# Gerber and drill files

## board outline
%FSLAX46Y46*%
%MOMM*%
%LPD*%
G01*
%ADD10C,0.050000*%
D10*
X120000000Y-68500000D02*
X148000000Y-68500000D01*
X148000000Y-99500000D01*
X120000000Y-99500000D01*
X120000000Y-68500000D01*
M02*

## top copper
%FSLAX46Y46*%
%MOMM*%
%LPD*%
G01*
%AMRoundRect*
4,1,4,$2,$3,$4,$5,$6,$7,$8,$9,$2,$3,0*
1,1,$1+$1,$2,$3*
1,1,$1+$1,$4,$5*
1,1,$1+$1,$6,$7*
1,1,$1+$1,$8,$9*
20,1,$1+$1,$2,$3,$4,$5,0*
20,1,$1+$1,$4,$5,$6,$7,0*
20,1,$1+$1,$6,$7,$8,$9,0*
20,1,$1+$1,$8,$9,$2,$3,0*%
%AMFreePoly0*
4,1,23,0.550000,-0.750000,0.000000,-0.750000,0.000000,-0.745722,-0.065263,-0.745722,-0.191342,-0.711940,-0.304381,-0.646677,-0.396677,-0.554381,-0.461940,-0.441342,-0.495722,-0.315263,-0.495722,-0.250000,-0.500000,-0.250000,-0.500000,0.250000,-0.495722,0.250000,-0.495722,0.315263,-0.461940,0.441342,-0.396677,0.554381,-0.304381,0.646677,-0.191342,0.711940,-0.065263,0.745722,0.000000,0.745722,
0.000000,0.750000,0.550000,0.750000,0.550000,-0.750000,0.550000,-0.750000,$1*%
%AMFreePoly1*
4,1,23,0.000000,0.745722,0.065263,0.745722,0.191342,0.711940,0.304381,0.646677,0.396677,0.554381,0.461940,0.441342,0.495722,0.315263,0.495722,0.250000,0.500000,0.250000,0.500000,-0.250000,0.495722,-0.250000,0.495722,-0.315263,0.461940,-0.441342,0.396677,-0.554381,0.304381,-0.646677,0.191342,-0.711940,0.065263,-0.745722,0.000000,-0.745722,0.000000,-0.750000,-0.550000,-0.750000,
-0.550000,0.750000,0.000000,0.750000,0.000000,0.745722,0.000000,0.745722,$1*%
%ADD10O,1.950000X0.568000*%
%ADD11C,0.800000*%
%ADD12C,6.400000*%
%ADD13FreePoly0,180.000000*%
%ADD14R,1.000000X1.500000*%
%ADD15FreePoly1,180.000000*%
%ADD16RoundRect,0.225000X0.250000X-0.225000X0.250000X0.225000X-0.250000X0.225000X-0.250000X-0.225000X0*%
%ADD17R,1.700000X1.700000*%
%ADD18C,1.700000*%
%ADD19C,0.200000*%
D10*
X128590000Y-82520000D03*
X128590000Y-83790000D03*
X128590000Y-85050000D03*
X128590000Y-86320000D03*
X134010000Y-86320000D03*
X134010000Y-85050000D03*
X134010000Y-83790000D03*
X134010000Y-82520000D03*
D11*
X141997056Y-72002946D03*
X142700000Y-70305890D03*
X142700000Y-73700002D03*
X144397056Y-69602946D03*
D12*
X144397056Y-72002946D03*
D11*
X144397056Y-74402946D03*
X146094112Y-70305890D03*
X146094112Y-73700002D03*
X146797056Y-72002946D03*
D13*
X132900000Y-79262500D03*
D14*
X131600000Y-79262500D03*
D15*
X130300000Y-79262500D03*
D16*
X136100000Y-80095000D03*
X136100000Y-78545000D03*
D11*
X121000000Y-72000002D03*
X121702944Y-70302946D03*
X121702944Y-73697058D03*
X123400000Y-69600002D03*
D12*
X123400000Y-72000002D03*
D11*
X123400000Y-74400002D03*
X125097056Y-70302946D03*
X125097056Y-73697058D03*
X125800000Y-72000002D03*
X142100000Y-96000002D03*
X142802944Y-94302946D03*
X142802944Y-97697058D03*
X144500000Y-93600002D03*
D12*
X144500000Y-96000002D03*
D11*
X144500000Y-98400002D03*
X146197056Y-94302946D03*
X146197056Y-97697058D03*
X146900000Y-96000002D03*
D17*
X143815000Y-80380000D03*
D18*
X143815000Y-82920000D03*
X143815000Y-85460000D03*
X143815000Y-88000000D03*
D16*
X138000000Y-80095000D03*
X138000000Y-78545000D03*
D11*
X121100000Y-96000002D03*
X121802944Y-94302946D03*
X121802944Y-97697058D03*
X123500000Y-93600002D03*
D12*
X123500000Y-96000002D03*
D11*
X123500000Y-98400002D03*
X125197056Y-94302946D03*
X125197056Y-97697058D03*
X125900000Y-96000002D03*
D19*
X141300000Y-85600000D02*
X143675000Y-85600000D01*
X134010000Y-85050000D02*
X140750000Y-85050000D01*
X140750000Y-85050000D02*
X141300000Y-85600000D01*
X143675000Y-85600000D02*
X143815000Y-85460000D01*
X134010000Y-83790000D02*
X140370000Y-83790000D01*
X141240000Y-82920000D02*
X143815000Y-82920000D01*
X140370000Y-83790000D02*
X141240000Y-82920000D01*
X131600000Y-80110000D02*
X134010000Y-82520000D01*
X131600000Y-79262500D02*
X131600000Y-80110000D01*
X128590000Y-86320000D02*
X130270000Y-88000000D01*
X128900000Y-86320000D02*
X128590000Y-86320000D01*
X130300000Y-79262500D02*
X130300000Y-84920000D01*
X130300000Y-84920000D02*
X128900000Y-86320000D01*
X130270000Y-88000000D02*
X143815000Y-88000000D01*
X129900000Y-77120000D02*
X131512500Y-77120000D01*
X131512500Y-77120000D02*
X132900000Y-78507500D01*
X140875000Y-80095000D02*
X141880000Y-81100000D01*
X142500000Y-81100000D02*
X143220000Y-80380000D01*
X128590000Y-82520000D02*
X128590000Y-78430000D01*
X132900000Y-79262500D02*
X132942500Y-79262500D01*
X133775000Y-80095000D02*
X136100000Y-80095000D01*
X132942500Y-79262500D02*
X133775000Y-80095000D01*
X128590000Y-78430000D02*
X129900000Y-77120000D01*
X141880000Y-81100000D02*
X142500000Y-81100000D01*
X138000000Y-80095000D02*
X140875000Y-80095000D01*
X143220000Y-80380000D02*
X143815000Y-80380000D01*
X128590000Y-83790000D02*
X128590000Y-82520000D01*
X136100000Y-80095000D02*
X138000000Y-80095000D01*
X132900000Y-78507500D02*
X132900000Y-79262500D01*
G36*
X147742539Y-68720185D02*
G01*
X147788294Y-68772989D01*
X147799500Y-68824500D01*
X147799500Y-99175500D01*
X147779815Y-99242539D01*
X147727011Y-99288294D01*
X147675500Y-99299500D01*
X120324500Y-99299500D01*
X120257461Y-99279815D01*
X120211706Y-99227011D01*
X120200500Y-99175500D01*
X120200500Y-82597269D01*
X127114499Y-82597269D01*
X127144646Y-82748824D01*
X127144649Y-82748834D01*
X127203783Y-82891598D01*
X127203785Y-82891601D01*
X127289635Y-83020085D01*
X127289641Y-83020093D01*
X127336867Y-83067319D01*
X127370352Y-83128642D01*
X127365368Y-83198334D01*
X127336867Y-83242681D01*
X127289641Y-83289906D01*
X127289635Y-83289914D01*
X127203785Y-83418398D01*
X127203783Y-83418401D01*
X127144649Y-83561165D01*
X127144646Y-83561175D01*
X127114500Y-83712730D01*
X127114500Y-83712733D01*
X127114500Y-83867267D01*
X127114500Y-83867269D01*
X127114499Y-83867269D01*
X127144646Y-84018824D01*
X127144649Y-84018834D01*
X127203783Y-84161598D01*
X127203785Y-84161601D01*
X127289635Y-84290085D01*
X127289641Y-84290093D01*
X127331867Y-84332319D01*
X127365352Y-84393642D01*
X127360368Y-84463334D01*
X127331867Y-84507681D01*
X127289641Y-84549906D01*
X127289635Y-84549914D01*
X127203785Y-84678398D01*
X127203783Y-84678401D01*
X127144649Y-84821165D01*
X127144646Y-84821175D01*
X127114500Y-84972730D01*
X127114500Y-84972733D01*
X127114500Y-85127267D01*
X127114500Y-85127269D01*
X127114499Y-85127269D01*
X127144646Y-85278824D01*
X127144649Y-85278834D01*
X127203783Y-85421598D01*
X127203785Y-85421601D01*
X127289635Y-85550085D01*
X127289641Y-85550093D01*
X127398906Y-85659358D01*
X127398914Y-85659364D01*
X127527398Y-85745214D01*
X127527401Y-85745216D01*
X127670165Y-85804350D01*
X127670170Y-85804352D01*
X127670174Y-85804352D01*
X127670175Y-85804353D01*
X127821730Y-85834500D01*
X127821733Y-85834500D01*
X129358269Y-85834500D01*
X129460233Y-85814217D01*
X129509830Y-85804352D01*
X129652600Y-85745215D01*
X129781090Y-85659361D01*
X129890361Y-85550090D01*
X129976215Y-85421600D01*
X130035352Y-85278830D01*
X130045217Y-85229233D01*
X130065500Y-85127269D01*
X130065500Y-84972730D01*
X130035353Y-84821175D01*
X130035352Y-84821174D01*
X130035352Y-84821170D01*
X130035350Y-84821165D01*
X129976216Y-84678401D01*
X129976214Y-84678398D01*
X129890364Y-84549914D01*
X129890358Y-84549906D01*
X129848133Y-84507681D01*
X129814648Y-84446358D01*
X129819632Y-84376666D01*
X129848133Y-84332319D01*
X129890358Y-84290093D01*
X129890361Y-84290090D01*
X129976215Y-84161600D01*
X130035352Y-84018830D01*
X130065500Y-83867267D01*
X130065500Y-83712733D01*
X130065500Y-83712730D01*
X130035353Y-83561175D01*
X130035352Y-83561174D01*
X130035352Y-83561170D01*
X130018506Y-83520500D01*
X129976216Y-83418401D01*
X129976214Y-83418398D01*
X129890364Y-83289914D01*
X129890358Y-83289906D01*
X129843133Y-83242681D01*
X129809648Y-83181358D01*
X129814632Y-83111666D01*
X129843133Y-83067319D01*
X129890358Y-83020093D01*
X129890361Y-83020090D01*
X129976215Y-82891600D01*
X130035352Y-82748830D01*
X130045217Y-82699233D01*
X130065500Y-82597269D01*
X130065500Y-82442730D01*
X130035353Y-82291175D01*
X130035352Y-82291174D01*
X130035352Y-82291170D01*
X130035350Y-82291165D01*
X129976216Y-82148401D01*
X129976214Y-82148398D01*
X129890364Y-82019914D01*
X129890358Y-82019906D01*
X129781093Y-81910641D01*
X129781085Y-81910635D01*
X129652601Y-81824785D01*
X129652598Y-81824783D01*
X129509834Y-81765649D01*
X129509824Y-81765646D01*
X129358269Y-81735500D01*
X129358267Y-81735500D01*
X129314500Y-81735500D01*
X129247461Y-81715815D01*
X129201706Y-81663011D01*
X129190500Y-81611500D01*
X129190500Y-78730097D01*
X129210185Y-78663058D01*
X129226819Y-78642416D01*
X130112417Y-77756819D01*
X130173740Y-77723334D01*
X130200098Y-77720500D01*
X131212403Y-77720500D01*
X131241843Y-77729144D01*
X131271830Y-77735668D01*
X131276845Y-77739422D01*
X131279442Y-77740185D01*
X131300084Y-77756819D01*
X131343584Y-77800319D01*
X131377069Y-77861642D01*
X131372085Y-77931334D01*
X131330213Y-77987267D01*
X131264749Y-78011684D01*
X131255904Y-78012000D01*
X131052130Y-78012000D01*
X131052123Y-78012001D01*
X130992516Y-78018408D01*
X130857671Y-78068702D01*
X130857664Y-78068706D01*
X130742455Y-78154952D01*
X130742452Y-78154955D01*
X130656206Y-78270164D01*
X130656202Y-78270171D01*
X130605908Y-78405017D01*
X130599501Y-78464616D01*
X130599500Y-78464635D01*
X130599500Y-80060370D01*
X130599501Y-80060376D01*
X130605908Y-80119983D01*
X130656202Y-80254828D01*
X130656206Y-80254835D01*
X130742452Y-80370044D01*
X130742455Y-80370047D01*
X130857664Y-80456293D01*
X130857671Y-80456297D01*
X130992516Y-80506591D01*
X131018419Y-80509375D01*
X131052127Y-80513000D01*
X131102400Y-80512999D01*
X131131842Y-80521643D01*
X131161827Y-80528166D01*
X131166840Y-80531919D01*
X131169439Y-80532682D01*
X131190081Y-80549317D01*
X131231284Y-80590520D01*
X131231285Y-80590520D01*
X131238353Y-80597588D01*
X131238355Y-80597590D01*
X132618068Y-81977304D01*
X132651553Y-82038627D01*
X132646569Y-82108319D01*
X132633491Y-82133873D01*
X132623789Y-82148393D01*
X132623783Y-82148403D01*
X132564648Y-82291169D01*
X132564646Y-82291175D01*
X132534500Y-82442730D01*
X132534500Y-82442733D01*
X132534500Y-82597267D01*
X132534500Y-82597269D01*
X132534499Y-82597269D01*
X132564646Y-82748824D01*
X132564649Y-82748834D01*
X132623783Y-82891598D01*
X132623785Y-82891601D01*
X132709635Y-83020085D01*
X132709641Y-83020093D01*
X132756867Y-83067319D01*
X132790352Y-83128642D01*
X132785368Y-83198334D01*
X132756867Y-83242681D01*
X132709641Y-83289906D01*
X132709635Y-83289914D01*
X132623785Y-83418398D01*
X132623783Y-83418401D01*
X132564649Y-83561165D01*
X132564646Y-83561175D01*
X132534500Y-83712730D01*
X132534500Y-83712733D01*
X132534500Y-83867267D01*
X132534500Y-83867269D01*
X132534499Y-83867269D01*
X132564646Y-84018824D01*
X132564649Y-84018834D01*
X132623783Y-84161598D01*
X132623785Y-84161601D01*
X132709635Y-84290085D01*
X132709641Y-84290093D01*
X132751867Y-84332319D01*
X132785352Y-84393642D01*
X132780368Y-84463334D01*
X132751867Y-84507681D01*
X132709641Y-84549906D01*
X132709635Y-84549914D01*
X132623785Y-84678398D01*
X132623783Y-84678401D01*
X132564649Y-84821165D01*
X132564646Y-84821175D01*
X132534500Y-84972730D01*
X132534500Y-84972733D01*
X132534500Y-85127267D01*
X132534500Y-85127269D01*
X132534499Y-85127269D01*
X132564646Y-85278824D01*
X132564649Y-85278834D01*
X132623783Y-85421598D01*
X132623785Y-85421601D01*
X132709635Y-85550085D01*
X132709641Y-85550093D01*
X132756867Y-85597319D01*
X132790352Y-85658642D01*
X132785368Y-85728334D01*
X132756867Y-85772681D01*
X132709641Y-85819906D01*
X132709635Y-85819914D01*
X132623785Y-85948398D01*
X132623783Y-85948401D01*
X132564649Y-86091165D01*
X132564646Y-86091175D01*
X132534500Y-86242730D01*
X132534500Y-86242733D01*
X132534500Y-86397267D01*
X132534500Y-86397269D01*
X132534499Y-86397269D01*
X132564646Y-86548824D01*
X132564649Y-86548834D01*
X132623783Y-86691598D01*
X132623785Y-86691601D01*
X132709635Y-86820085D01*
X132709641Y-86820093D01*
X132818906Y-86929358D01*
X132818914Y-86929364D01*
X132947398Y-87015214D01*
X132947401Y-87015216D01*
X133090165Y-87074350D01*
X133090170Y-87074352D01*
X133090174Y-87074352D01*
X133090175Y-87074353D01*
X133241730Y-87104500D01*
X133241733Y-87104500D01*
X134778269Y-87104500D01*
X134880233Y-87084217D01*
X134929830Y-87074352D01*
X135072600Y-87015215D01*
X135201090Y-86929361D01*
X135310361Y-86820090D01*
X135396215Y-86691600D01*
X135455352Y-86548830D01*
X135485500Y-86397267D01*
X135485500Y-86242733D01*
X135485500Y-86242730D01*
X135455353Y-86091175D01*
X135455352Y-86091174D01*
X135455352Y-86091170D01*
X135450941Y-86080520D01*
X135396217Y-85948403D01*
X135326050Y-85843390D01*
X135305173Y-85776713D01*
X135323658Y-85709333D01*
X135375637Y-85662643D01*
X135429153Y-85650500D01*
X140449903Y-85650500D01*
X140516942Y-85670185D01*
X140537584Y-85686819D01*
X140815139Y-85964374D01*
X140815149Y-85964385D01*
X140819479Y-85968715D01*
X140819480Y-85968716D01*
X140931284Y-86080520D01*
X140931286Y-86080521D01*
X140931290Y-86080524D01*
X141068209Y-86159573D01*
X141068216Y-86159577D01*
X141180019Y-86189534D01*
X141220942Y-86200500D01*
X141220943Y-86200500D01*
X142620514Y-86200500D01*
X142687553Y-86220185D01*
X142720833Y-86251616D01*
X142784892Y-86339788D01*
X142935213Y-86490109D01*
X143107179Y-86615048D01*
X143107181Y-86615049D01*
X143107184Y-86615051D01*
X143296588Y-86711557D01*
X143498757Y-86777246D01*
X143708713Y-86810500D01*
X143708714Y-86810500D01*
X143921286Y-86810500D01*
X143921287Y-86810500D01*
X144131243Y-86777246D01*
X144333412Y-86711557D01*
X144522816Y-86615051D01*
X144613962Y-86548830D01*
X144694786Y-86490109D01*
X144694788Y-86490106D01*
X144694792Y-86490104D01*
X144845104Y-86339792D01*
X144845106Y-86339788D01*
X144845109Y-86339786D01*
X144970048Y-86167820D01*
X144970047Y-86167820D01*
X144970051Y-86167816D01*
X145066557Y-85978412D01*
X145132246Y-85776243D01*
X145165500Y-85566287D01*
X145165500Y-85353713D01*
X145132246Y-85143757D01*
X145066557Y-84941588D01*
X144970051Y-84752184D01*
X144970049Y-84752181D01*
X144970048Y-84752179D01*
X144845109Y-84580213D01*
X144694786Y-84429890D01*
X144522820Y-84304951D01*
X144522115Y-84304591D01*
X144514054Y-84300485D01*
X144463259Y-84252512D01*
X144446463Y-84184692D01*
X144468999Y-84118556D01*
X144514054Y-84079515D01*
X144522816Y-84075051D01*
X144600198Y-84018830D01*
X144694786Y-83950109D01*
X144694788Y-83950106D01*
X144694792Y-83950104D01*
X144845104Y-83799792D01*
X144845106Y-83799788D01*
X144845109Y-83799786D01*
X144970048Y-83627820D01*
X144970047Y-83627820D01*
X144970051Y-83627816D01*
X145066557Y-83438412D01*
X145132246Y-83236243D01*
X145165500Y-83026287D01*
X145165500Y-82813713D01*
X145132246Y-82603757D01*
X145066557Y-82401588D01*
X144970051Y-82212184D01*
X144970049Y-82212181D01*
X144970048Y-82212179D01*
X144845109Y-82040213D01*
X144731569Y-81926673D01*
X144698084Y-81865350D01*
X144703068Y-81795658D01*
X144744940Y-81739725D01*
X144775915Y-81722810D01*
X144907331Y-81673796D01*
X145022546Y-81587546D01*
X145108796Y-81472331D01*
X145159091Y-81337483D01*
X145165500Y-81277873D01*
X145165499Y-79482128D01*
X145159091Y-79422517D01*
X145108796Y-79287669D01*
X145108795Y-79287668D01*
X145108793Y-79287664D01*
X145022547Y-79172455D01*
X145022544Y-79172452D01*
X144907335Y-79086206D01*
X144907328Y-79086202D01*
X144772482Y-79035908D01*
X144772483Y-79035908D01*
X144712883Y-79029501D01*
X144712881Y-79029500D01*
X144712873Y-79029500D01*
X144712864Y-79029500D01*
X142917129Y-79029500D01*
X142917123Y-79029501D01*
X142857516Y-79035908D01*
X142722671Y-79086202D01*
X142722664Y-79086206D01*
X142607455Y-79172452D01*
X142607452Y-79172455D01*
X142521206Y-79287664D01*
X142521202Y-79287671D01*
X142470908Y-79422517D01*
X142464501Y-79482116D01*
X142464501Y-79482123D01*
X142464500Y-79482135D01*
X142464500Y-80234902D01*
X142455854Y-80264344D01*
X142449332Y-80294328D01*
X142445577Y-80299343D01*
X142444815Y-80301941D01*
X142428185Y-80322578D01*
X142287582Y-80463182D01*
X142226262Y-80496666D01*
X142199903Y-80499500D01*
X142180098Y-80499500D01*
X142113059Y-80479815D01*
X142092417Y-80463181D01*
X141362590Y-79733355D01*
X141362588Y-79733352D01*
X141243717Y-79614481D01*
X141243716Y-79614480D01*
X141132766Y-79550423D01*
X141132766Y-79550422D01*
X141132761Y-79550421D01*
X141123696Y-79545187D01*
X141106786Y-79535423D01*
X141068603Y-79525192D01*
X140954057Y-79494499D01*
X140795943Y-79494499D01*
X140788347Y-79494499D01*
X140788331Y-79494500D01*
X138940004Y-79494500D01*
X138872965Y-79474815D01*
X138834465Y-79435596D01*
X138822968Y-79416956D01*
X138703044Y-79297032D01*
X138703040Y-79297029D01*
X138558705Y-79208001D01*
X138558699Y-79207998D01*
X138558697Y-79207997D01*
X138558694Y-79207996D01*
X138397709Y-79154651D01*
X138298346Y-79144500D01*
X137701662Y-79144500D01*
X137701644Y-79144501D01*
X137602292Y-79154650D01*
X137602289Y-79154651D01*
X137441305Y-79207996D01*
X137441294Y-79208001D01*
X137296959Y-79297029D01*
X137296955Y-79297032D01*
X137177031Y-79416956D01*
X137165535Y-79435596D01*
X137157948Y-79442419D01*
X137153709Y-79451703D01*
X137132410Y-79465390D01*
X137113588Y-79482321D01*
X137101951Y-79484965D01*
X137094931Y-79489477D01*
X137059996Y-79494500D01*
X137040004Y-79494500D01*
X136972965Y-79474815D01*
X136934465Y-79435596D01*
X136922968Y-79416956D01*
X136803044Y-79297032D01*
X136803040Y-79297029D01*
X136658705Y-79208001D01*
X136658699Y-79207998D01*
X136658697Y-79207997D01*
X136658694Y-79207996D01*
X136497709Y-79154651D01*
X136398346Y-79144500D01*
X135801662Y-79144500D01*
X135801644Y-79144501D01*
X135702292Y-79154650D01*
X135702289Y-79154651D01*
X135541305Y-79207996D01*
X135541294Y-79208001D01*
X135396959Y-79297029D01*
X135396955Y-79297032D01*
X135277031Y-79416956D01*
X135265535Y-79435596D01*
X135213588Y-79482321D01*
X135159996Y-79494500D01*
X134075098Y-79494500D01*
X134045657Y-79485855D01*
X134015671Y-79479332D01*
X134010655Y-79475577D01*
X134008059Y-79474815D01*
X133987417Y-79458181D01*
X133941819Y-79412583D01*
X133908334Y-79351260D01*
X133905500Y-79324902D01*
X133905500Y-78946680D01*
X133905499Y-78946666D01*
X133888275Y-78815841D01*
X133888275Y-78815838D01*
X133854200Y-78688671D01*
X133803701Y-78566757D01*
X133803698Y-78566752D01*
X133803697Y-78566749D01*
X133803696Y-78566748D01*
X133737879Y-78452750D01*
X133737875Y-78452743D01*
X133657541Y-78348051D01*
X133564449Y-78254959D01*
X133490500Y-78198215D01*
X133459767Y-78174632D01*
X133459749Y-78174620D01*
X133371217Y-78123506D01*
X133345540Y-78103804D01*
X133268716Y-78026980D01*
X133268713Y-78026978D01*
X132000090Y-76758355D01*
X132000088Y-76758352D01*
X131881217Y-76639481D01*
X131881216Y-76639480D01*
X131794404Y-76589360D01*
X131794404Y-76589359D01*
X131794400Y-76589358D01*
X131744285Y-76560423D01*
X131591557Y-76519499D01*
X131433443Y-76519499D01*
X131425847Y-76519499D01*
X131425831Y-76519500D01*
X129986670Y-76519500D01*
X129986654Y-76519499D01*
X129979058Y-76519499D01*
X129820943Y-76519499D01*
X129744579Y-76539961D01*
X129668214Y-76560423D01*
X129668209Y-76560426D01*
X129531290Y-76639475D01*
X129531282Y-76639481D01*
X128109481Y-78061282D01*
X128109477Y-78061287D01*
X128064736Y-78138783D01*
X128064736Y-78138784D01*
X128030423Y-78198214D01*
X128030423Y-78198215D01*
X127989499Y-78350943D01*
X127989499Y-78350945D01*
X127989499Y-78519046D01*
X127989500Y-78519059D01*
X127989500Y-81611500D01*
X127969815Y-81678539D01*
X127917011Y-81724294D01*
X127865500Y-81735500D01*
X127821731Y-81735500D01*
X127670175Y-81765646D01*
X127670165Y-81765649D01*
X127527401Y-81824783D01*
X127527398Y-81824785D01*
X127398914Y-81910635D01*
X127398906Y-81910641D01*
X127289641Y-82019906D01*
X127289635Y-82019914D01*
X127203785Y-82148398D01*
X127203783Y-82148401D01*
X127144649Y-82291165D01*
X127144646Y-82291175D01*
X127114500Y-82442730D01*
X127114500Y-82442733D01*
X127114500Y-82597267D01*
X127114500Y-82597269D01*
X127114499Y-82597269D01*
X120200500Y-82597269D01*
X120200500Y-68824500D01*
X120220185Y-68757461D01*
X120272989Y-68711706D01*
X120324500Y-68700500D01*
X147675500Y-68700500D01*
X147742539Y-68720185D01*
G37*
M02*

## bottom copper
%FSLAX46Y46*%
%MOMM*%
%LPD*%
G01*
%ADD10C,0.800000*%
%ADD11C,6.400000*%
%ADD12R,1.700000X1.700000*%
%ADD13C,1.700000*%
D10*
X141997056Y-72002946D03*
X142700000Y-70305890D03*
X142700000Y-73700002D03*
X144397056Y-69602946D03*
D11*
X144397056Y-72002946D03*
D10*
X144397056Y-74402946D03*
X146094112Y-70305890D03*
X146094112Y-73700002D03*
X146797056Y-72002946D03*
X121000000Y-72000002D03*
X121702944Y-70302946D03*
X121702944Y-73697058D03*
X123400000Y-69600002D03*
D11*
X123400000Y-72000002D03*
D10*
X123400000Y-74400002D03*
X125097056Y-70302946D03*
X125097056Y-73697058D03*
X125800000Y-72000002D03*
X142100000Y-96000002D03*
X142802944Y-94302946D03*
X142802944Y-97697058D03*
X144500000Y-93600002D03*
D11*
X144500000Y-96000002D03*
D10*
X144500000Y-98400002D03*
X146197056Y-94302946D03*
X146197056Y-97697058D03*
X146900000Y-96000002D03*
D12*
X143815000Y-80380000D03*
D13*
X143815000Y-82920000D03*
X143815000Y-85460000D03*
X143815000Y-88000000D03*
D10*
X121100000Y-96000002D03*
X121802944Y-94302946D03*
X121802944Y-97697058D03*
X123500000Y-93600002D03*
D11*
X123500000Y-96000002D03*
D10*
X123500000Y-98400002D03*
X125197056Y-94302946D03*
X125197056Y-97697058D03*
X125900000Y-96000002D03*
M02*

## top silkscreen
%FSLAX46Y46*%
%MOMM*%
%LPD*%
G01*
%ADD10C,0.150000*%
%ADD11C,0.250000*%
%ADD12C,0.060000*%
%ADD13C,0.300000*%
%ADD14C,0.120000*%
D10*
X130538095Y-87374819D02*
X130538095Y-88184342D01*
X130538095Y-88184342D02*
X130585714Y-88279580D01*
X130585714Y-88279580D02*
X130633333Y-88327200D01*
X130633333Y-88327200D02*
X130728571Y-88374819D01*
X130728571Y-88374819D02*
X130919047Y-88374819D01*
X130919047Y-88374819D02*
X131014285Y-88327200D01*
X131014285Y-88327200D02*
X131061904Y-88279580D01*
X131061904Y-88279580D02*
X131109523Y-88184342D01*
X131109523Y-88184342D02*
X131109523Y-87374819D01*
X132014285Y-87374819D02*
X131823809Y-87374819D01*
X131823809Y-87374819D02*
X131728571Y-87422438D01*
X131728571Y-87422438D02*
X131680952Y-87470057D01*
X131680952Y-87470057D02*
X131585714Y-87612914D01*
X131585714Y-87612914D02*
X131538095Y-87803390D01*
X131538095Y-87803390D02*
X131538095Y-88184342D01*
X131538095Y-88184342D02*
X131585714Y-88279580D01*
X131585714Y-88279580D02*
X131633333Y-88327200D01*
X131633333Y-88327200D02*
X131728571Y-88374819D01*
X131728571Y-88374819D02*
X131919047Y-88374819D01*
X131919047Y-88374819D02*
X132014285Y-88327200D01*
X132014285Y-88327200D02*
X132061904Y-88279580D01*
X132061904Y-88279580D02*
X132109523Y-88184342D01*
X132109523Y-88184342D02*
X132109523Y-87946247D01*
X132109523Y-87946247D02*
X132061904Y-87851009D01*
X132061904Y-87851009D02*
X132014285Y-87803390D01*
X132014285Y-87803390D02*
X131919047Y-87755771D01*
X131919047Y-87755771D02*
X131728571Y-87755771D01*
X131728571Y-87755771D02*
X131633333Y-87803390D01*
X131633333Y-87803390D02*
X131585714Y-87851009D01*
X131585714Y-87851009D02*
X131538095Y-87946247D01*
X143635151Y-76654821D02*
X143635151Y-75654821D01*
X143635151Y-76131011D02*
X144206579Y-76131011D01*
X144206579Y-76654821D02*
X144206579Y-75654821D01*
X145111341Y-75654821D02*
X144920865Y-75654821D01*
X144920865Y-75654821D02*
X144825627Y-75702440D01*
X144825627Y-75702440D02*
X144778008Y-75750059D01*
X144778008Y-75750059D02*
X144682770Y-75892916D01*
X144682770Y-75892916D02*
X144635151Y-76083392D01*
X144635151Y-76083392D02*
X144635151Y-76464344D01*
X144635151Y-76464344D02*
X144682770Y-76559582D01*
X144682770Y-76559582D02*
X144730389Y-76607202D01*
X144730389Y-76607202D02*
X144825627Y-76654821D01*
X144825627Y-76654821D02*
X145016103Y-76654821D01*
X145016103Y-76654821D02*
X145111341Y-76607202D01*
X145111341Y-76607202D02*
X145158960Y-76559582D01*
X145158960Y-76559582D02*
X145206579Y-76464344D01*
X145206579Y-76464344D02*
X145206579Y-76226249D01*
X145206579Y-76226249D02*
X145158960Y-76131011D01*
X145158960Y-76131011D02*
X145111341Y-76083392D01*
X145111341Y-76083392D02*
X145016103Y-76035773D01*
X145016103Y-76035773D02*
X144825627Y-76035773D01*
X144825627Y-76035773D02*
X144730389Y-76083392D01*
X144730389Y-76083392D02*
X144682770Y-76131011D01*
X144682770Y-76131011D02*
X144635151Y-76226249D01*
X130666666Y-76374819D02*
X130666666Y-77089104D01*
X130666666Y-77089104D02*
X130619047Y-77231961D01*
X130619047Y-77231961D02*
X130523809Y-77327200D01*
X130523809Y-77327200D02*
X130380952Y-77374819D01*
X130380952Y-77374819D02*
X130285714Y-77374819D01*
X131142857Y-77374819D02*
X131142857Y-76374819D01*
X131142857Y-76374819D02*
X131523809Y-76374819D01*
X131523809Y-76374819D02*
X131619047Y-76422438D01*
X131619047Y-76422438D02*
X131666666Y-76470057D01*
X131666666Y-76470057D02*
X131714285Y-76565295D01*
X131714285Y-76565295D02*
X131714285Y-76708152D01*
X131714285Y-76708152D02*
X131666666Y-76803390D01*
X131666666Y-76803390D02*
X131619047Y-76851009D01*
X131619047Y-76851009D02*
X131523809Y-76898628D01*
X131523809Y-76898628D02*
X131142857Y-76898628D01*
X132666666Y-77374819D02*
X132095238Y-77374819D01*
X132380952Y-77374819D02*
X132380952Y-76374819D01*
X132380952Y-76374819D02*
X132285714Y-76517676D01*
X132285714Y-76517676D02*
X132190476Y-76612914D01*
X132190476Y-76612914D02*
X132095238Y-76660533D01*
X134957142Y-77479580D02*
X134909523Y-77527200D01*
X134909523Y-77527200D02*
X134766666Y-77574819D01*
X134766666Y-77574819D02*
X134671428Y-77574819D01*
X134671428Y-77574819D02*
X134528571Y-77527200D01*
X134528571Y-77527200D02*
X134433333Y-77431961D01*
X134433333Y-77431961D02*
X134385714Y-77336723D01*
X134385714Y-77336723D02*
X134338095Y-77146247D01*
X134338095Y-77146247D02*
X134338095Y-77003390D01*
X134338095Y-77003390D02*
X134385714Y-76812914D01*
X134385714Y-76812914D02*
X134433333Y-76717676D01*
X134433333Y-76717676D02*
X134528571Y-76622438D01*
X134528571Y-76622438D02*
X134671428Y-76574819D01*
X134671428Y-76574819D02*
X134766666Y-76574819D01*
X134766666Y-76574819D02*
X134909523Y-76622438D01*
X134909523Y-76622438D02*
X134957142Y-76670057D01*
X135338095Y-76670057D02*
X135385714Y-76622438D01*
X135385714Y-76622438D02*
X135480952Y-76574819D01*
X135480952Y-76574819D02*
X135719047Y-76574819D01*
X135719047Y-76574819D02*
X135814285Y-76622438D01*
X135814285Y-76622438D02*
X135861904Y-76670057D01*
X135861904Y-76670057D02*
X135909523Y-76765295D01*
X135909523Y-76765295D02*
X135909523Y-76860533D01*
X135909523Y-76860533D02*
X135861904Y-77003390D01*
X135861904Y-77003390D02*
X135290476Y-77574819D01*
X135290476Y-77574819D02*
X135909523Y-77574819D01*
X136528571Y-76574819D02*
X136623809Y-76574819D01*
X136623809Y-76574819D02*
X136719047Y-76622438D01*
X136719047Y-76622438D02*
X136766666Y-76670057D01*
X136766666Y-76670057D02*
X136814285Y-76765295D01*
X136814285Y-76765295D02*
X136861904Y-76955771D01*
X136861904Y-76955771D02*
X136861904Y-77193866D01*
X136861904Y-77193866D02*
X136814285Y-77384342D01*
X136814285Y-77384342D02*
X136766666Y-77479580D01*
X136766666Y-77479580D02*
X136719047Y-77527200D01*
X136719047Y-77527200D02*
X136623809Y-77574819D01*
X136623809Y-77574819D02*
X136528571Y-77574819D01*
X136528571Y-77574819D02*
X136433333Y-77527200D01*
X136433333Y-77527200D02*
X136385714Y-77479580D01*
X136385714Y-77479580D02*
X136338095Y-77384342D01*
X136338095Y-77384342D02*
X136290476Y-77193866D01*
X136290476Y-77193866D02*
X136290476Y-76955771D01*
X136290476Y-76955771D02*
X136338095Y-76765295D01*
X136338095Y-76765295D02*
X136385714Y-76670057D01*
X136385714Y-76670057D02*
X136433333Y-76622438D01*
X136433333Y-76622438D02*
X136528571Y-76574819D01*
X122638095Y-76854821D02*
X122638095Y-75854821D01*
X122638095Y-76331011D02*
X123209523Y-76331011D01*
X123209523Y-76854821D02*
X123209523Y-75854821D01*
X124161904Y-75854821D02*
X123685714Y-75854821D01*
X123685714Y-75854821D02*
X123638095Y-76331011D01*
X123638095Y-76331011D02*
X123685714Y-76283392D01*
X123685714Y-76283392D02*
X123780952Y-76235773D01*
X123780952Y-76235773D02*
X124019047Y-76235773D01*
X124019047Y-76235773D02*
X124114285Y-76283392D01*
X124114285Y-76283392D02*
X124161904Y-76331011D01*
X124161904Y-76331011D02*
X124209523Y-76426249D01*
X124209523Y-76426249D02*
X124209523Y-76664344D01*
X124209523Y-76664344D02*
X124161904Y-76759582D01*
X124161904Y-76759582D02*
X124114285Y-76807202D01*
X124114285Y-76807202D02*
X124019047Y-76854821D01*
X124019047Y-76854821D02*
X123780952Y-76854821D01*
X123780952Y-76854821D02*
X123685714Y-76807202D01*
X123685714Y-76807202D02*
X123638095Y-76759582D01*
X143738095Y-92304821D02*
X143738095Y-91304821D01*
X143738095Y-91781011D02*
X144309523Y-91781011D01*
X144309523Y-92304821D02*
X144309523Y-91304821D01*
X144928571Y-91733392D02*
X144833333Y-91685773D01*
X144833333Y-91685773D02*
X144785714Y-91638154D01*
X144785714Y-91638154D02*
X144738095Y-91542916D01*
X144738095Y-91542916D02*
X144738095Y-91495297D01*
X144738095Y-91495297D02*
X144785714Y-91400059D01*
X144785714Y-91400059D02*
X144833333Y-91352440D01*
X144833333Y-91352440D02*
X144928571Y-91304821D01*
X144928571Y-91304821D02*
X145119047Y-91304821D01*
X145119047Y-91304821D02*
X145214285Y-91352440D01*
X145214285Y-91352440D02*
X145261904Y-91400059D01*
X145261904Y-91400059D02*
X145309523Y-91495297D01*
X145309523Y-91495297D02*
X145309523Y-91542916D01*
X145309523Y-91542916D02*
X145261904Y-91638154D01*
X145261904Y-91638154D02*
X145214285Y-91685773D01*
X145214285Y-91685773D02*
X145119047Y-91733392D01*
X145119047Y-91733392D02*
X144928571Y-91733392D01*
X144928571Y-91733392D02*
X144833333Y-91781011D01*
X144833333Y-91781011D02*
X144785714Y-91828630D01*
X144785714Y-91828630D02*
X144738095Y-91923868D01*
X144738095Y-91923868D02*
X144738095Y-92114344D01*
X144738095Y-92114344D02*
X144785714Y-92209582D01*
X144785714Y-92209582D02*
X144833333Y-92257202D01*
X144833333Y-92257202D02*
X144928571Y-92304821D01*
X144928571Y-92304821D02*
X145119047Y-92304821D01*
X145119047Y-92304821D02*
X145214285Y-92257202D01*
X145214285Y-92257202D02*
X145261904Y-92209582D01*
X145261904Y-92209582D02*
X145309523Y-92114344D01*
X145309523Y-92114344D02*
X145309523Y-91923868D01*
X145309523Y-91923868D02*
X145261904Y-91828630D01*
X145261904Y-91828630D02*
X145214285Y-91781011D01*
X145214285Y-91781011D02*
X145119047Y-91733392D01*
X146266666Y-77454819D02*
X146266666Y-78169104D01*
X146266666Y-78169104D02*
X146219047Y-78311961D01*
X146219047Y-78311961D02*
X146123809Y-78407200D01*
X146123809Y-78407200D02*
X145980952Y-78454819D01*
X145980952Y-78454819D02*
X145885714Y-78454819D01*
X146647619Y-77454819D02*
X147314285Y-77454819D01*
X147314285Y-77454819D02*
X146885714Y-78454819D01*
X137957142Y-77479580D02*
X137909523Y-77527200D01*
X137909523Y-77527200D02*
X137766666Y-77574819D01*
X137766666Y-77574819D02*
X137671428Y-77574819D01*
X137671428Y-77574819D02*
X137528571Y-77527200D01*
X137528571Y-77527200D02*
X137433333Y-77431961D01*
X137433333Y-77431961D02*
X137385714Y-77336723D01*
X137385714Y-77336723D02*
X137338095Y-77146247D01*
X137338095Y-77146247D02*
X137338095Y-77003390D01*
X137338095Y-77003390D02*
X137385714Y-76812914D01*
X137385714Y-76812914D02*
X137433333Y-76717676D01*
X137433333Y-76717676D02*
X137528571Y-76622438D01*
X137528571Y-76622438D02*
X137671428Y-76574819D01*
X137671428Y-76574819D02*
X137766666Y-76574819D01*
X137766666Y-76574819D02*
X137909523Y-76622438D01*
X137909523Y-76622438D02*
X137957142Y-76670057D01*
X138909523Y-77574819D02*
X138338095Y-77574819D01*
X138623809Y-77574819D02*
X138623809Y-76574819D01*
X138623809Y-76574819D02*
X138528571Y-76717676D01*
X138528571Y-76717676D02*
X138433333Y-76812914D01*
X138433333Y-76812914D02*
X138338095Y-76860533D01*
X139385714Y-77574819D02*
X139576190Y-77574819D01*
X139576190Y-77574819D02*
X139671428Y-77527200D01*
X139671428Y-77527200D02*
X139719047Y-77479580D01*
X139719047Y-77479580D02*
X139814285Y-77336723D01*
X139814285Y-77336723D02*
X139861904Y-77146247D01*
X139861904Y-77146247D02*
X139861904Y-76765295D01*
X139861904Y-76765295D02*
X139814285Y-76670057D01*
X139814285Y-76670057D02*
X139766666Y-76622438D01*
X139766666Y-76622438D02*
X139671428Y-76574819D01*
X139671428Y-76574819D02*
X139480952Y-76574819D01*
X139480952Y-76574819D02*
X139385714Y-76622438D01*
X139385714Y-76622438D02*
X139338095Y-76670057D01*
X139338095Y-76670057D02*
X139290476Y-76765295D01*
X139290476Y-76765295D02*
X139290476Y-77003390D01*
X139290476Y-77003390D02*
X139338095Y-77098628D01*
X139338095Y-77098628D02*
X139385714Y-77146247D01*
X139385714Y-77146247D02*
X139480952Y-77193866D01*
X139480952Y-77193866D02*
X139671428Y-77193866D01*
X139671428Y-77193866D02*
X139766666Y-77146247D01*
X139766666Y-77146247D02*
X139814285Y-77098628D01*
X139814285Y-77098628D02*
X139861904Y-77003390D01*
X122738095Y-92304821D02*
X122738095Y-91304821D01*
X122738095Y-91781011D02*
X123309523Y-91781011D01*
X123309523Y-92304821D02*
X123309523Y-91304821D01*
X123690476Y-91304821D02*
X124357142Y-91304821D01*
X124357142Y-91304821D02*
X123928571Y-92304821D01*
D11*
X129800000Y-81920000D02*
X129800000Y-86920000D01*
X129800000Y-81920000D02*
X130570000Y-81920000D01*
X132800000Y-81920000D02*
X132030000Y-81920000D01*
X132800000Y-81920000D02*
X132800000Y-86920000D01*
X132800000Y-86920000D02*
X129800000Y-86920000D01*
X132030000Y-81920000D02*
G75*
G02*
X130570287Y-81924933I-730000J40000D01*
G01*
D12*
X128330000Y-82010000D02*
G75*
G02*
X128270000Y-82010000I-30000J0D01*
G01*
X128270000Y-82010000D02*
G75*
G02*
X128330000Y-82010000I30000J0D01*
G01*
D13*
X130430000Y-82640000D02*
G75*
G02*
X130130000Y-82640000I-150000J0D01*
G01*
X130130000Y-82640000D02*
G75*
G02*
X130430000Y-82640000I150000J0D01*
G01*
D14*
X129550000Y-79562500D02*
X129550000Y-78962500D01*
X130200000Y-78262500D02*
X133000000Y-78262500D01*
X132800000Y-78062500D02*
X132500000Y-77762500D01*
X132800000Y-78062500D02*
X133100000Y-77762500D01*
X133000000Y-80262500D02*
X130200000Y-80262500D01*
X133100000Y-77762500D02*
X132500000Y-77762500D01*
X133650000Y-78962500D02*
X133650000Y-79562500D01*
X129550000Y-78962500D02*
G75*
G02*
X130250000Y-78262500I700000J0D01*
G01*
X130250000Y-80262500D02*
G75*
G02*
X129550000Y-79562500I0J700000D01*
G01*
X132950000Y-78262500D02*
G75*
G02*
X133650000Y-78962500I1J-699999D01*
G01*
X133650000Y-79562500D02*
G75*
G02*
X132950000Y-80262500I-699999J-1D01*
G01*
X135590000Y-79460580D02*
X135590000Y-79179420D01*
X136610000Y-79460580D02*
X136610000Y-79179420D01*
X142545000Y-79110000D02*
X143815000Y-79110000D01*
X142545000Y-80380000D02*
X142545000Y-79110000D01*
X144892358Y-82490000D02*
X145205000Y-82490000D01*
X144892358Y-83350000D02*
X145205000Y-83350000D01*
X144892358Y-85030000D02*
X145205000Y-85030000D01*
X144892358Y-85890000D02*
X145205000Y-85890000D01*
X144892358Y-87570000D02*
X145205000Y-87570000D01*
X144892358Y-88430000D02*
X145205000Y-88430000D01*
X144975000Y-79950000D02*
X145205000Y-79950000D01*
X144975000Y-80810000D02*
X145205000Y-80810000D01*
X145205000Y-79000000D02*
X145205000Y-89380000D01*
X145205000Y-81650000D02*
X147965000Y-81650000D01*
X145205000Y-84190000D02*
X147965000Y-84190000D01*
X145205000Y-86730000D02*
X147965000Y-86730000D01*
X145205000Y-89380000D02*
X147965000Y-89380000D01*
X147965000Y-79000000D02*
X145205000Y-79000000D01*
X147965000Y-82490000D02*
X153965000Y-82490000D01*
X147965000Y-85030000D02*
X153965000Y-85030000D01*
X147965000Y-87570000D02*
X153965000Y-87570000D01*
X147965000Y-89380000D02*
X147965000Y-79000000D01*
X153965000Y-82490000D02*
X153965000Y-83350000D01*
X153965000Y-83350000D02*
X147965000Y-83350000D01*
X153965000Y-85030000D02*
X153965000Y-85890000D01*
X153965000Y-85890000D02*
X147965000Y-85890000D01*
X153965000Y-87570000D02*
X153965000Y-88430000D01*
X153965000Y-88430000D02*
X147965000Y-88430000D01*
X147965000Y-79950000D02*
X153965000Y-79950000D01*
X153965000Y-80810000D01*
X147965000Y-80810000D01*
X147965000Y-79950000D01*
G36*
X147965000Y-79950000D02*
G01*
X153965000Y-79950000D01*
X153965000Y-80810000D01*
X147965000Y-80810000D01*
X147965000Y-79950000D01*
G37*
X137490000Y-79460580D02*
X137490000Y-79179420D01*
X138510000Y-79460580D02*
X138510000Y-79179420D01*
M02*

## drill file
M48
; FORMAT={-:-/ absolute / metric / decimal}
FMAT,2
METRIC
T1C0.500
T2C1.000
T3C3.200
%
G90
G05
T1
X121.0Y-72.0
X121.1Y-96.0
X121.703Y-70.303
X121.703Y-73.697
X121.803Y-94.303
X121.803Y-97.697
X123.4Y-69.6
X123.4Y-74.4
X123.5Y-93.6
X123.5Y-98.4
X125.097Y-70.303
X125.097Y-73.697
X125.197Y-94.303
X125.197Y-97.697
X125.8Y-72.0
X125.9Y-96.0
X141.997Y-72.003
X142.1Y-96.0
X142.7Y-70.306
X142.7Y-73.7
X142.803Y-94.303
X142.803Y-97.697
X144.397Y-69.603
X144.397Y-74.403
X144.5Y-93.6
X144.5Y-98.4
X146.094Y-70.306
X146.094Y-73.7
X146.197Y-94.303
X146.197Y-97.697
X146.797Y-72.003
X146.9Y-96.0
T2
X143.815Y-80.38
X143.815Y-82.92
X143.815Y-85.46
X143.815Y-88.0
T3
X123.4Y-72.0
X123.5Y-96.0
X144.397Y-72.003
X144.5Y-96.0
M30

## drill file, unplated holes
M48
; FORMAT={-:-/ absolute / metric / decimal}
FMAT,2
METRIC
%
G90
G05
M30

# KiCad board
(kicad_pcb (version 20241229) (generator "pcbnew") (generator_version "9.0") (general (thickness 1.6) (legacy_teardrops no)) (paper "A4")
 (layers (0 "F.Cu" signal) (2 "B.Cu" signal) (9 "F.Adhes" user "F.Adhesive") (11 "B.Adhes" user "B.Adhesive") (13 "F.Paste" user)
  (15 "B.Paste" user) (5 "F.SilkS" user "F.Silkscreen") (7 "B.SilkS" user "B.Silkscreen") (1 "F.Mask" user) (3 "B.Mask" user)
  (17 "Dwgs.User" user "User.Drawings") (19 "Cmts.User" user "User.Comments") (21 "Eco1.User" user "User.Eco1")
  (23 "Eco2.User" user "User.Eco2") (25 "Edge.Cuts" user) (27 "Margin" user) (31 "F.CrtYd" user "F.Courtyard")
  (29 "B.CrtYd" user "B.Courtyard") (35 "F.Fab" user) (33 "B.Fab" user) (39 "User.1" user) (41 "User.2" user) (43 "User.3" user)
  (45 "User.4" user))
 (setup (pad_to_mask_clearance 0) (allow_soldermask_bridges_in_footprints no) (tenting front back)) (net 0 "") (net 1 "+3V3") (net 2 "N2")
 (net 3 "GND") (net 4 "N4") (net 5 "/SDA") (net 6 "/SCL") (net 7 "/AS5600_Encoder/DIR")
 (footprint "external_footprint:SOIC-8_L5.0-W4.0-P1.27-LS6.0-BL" (layer "F.Cu") (at 131.3 84.42 -90)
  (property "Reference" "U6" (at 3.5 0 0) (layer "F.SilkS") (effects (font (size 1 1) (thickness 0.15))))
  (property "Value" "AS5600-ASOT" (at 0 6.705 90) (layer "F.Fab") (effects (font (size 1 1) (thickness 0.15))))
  (fp_line (start -2.5 1.5) (end 2.5 1.5) (stroke (width 0.25) (type solid)) (layer "F.SilkS"))
  (fp_line (start -2.5 1.5) (end -2.5 0.73) (stroke (width 0.25) (type solid)) (layer "F.SilkS"))
  (fp_line (start -2.5 -1.5) (end -2.5 -0.73) (stroke (width 0.25) (type solid)) (layer "F.SilkS"))
  (fp_line (start -2.5 -1.5) (end 2.5 -1.5) (stroke (width 0.25) (type solid)) (layer "F.SilkS"))
  (fp_line (start 2.5 -1.5) (end 2.5 1.5) (stroke (width 0.25) (type solid)) (layer "F.SilkS"))
  (fp_arc (start -2.5 -0.73) (mid -1.808909 -0.002471) (end -2.495067 0.729713) (stroke (width 0.25) (type solid)) (layer "F.SilkS"))
  (fp_circle (center -2.41 3) (end -2.38 3) (stroke (width 0.06) (type solid)) (fill no) (layer "F.SilkS"))
  (fp_circle (center -1.78 1.02) (end -1.63 1.02) (stroke (width 0.3) (type solid)) (fill no) (layer "F.SilkS"))
  (pad "1" smd oval (at -1.9 2.71 270) (size 0.568 1.95) (layers "F.Cu" "F.Mask" "F.Paste") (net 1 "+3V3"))
  (pad "2" smd oval (at -0.63 2.71 270) (size 0.568 1.95) (layers "F.Cu" "F.Mask" "F.Paste") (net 1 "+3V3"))
  (pad "3" smd oval (at 0.63 2.71 270) (size 0.568 1.95) (layers "F.Cu" "F.Mask" "F.Paste") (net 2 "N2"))
  (pad "4" smd oval (at 1.9 2.71 270) (size 0.568 1.95) (layers "F.Cu" "F.Mask" "F.Paste") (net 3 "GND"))
  (pad "5" smd oval (at 1.9 -2.71 270) (size 0.568 1.95) (layers "F.Cu" "F.Mask" "F.Paste") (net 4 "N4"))
  (pad "6" smd oval (at 0.63 -2.71 270) (size 0.568 1.95) (layers "F.Cu" "F.Mask" "F.Paste") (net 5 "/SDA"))
  (pad "7" smd oval (at -0.63 -2.71 270) (size 0.568 1.95) (layers "F.Cu" "F.Mask" "F.Paste") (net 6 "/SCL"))
  (pad "8" smd oval (at -1.9 -2.71 270) (size 0.568 1.95) (layers "F.Cu" "F.Mask" "F.Paste") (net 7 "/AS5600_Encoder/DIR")))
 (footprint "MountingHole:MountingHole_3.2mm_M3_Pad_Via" (layer "F.Cu") (at 144.397056 72.002946)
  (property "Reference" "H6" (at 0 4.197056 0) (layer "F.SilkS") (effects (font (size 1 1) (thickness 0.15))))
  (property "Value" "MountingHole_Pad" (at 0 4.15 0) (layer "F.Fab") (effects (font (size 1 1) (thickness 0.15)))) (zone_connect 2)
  (pad "1" thru_hole circle (at -2.4 0) (size 0.8 0.8) (drill 0.5) (layers "*.Cu" "*.Mask") (remove_unused_layers no) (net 3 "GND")
   (zone_connect 2))
  (pad "1" thru_hole circle (at -1.697056 -1.697056) (size 0.8 0.8) (drill 0.5) (layers "*.Cu" "*.Mask") (remove_unused_layers no)
   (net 3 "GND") (zone_connect 2))
  (pad "1" thru_hole circle (at -1.697056 1.697056) (size 0.8 0.8) (drill 0.5) (layers "*.Cu" "*.Mask") (remove_unused_layers no)
   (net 3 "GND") (zone_connect 2))
  (pad "1" thru_hole circle (at 0 -2.4) (size 0.8 0.8) (drill 0.5) (layers "*.Cu" "*.Mask") (remove_unused_layers no) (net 3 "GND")
   (zone_connect 2))
  (pad "1" thru_hole circle (at 0 0) (size 6.4 6.4) (drill 3.2) (layers "*.Cu" "*.Mask") (remove_unused_layers no) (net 3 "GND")
   (zone_connect 2))
  (pad "1" thru_hole circle (at 0 2.4) (size 0.8 0.8) (drill 0.5) (layers "*.Cu" "*.Mask") (remove_unused_layers no) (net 3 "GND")
   (zone_connect 2))
  (pad "1" thru_hole circle (at 1.697056 -1.697056) (size 0.8 0.8) (drill 0.5) (layers "*.Cu" "*.Mask") (remove_unused_layers no)
   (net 3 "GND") (zone_connect 2))
  (pad "1" thru_hole circle (at 1.697056 1.697056) (size 0.8 0.8) (drill 0.5) (layers "*.Cu" "*.Mask") (remove_unused_layers no)
   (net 3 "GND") (zone_connect 2))
  (pad "1" thru_hole circle (at 2.4 0) (size 0.8 0.8) (drill 0.5) (layers "*.Cu" "*.Mask") (remove_unused_layers no) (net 3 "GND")
   (zone_connect 2)))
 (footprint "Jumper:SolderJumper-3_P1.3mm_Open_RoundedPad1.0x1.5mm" (layer "F.Cu") (at 131.6 79.2625 180)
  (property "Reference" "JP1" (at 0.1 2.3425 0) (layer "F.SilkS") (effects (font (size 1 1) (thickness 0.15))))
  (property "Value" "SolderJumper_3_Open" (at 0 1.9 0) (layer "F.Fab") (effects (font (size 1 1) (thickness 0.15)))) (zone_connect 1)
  (fp_line (start 2.05 -0.3) (end 2.05 0.3) (stroke (width 0.12) (type solid)) (layer "F.SilkS"))
  (fp_line (start 1.4 1) (end -1.4 1) (stroke (width 0.12) (type solid)) (layer "F.SilkS"))
  (fp_line (start -1.2 1.2) (end -0.9 1.5) (stroke (width 0.12) (type solid)) (layer "F.SilkS"))
  (fp_line (start -1.2 1.2) (end -1.5 1.5) (stroke (width 0.12) (type solid)) (layer "F.SilkS"))
  (fp_line (start -1.4 -1) (end 1.4 -1) (stroke (width 0.12) (type solid)) (layer "F.SilkS"))
  (fp_line (start -1.5 1.5) (end -0.9 1.5) (stroke (width 0.12) (type solid)) (layer "F.SilkS"))
  (fp_line (start -2.05 0.3) (end -2.05 -0.3) (stroke (width 0.12) (type solid)) (layer "F.SilkS"))
  (fp_arc (start 2.05 0.3) (mid 1.844975 0.794975) (end 1.35 1) (stroke (width 0.12) (type solid)) (layer "F.SilkS"))
  (fp_arc (start 1.35 -1) (mid 1.844975 -0.794975) (end 2.05 -0.3) (stroke (width 0.12) (type solid)) (layer "F.SilkS"))
  (fp_arc (start -1.35 1) (mid -1.844975 0.794975) (end -2.05 0.3) (stroke (width 0.12) (type solid)) (layer "F.SilkS"))
  (fp_arc (start -2.05 -0.3) (mid -1.844975 -0.794975) (end -1.35 -1) (stroke (width 0.12) (type solid)) (layer "F.SilkS"))
  (pad "1" smd custom (at -1.3 0 180) (size 1 0.5) (layers "F.Cu" "F.Mask") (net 1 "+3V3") (zone_connect 2) (thermal_bridge_angle 45)
   (options (clearance outline) (anchor rect)) (primitives))
  (pad "2" smd rect (at 0 0 180) (size 1 1.5) (layers "F.Cu" "F.Mask") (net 7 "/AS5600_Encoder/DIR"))
  (pad "3" smd custom (at 1.3 0 180) (size 1 0.5) (layers "F.Cu" "F.Mask") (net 3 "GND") (zone_connect 2) (thermal_bridge_angle 45)
   (options (clearance outline) (anchor rect)) (primitives)))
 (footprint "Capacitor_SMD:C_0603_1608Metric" (layer "F.Cu") (at 136.1 79.32 90)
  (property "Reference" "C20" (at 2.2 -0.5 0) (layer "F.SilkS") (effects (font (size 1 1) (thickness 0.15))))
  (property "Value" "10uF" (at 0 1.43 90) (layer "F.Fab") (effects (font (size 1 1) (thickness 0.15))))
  (fp_line (start -0.14058 -0.51) (end 0.14058 -0.51) (stroke (width 0.12) (type solid)) (layer "F.SilkS"))
  (fp_line (start -0.14058 0.51) (end 0.14058 0.51) (stroke (width 0.12) (type solid)) (layer "F.SilkS"))
  (pad "1" smd roundrect (at -0.775 0 90) (size 0.9 0.95) (layers "F.Cu" "F.Mask" "F.Paste") (roundrect_rratio 0.25) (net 1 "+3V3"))
  (pad "2" smd roundrect (at 0.775 0 90) (size 0.9 0.95) (layers "F.Cu" "F.Mask" "F.Paste") (roundrect_rratio 0.25) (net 3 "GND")))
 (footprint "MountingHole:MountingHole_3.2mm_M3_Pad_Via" (layer "F.Cu") (at 123.4 72.000002)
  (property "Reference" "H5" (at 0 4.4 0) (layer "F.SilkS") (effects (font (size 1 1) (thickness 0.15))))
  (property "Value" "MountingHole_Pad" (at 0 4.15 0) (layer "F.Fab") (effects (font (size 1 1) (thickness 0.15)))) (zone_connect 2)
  (pad "1" thru_hole circle (at -2.4 0) (size 0.8 0.8) (drill 0.5) (layers "*.Cu" "*.Mask") (remove_unused_layers no) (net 3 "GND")
   (zone_connect 2))
  (pad "1" thru_hole circle (at -1.697056 -1.697056) (size 0.8 0.8) (drill 0.5) (layers "*.Cu" "*.Mask") (remove_unused_layers no)
   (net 3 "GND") (zone_connect 2))
  (pad "1" thru_hole circle (at -1.697056 1.697056) (size 0.8 0.8) (drill 0.5) (layers "*.Cu" "*.Mask") (remove_unused_layers no)
   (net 3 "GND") (zone_connect 2))
  (pad "1" thru_hole circle (at 0 -2.4) (size 0.8 0.8) (drill 0.5) (layers "*.Cu" "*.Mask") (remove_unused_layers no) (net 3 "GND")
   (zone_connect 2))
  (pad "1" thru_hole circle (at 0 0) (size 6.4 6.4) (drill 3.2) (layers "*.Cu" "*.Mask") (remove_unused_layers no) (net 3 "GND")
   (zone_connect 2))
  (pad "1" thru_hole circle (at 0 2.4) (size 0.8 0.8) (drill 0.5) (layers "*.Cu" "*.Mask") (remove_unused_layers no) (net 3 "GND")
   (zone_connect 2))
  (pad "1" thru_hole circle (at 1.697056 -1.697056) (size 0.8 0.8) (drill 0.5) (layers "*.Cu" "*.Mask") (remove_unused_layers no)
   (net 3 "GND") (zone_connect 2))
  (pad "1" thru_hole circle (at 1.697056 1.697056) (size 0.8 0.8) (drill 0.5) (layers "*.Cu" "*.Mask") (remove_unused_layers no)
   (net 3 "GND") (zone_connect 2))
  (pad "1" thru_hole circle (at 2.4 0) (size 0.8 0.8) (drill 0.5) (layers "*.Cu" "*.Mask") (remove_unused_layers no) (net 3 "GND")
   (zone_connect 2)))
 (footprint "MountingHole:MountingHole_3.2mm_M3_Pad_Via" (layer "F.Cu") (at 144.5 96.000002)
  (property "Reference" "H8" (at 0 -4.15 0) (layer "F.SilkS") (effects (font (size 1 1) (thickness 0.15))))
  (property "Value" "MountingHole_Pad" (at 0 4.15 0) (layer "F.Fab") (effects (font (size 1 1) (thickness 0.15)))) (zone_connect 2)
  (pad "1" thru_hole circle (at -2.4 0) (size 0.8 0.8) (drill 0.5) (layers "*.Cu" "*.Mask") (remove_unused_layers no) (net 3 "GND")
   (zone_connect 2))
  (pad "1" thru_hole circle (at -1.697056 -1.697056) (size 0.8 0.8) (drill 0.5) (layers "*.Cu" "*.Mask") (remove_unused_layers no)
   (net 3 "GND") (zone_connect 2))
  (pad "1" thru_hole circle (at -1.697056 1.697056) (size 0.8 0.8) (drill 0.5) (layers "*.Cu" "*.Mask") (remove_unused_layers no)
   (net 3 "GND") (zone_connect 2))
  (pad "1" thru_hole circle (at 0 -2.4) (size 0.8 0.8) (drill 0.5) (layers "*.Cu" "*.Mask") (remove_unused_layers no) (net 3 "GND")
   (zone_connect 2))
  (pad "1" thru_hole circle (at 0 0) (size 6.4 6.4) (drill 3.2) (layers "*.Cu" "*.Mask") (remove_unused_layers no) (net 3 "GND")
   (zone_connect 2))
  (pad "1" thru_hole circle (at 0 2.4) (size 0.8 0.8) (drill 0.5) (layers "*.Cu" "*.Mask") (remove_unused_layers no) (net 3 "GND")
   (zone_connect 2))
  (pad "1" thru_hole circle (at 1.697056 -1.697056) (size 0.8 0.8) (drill 0.5) (layers "*.Cu" "*.Mask") (remove_unused_layers no)
   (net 3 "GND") (zone_connect 2))
  (pad "1" thru_hole circle (at 1.697056 1.697056) (size 0.8 0.8) (drill 0.5) (layers "*.Cu" "*.Mask") (remove_unused_layers no)
   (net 3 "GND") (zone_connect 2))
  (pad "1" thru_hole circle (at 2.4 0) (size 0.8 0.8) (drill 0.5) (layers "*.Cu" "*.Mask") (remove_unused_layers no) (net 3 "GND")
   (zone_connect 2)))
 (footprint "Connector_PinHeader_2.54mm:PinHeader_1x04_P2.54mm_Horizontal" (layer "F.Cu") (at 143.815 80.38)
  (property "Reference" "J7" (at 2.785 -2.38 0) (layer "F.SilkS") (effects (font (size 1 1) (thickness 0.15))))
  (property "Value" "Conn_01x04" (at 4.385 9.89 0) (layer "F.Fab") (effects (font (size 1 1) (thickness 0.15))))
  (fp_line (start -1.27 -1.27) (end 0 -1.27) (stroke (width 0.12) (type solid)) (layer "F.SilkS"))
  (fp_line (start -1.27 0) (end -1.27 -1.27) (stroke (width 0.12) (type solid)) (layer "F.SilkS"))
  (fp_line (start 1.077358 2.11) (end 1.39 2.11) (stroke (width 0.12) (type solid)) (layer "F.SilkS"))
  (fp_line (start 1.077358 2.97) (end 1.39 2.97) (stroke (width 0.12) (type solid)) (layer "F.SilkS"))
  (fp_line (start 1.077358 4.65) (end 1.39 4.65) (stroke (width 0.12) (type solid)) (layer "F.SilkS"))
  (fp_line (start 1.077358 5.51) (end 1.39 5.51) (stroke (width 0.12) (type solid)) (layer "F.SilkS"))
  (fp_line (start 1.077358 7.19) (end 1.39 7.19) (stroke (width 0.12) (type solid)) (layer "F.SilkS"))
  (fp_line (start 1.077358 8.05) (end 1.39 8.05) (stroke (width 0.12) (type solid)) (layer "F.SilkS"))
  (fp_line (start 1.16 -0.43) (end 1.39 -0.43) (stroke (width 0.12) (type solid)) (layer "F.SilkS"))
  (fp_line (start 1.16 0.43) (end 1.39 0.43) (stroke (width 0.12) (type solid)) (layer "F.SilkS"))
  (fp_line (start 1.39 -1.38) (end 1.39 9) (stroke (width 0.12) (type solid)) (layer "F.SilkS"))
  (fp_line (start 1.39 1.27) (end 4.15 1.27) (stroke (width 0.12) (type solid)) (layer "F.SilkS"))
  (fp_line (start 1.39 3.81) (end 4.15 3.81) (stroke (width 0.12) (type solid)) (layer "F.SilkS"))
  (fp_line (start 1.39 6.35) (end 4.15 6.35) (stroke (width 0.12) (type solid)) (layer "F.SilkS"))
  (fp_line (start 1.39 9) (end 4.15 9) (stroke (width 0.12) (type solid)) (layer "F.SilkS"))
  (fp_line (start 4.15 -1.38) (end 1.39 -1.38) (stroke (width 0.12) (type solid)) (layer "F.SilkS"))
  (fp_line (start 4.15 2.11) (end 10.15 2.11) (stroke (width 0.12) (type solid)) (layer "F.SilkS"))
  (fp_line (start 4.15 4.65) (end 10.15 4.65) (stroke (width 0.12) (type solid)) (layer "F.SilkS"))
  (fp_line (start 4.15 7.19) (end 10.15 7.19) (stroke (width 0.12) (type solid)) (layer "F.SilkS"))
  (fp_line (start 4.15 9) (end 4.15 -1.38) (stroke (width 0.12) (type solid)) (layer "F.SilkS"))
  (fp_line (start 10.15 2.11) (end 10.15 2.97) (stroke (width 0.12) (type solid)) (layer "F.SilkS"))
  (fp_line (start 10.15 2.97) (end 4.15 2.97) (stroke (width 0.12) (type solid)) (layer "F.SilkS"))
  (fp_line (start 10.15 4.65) (end 10.15 5.51) (stroke (width 0.12) (type solid)) (layer "F.SilkS"))
  (fp_line (start 10.15 5.51) (end 4.15 5.51) (stroke (width 0.12) (type solid)) (layer "F.SilkS"))
  (fp_line (start 10.15 7.19) (end 10.15 8.05) (stroke (width 0.12) (type solid)) (layer "F.SilkS"))
  (fp_line (start 10.15 8.05) (end 4.15 8.05) (stroke (width 0.12) (type solid)) (layer "F.SilkS"))
  (fp_rect (start 4.15 -0.43) (end 10.15 0.43) (stroke (width 0.12) (type solid)) (fill yes) (layer "F.SilkS"))
  (pad "1" thru_hole rect (at 0 0) (size 1.7 1.7) (drill 1) (layers "*.Cu" "*.Mask") (remove_unused_layers no) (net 1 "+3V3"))
  (pad "2" thru_hole circle (at 0 2.54) (size 1.7 1.7) (drill 1) (layers "*.Cu" "*.Mask") (remove_unused_layers no) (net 6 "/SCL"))
  (pad "3" thru_hole circle (at 0 5.08) (size 1.7 1.7) (drill 1) (layers "*.Cu" "*.Mask") (remove_unused_layers no) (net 5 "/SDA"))
  (pad "4" thru_hole circle (at 0 7.62) (size 1.7 1.7) (drill 1) (layers "*.Cu" "*.Mask") (remove_unused_layers no) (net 3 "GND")))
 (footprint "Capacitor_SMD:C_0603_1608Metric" (layer "F.Cu") (at 138 79.32 90)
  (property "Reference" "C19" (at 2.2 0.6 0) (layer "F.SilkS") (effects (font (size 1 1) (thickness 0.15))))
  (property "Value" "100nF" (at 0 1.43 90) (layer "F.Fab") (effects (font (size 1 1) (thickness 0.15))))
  (fp_line (start -0.14058 -0.51) (end 0.14058 -0.51) (stroke (width 0.12) (type solid)) (layer "F.SilkS"))
  (fp_line (start -0.14058 0.51) (end 0.14058 0.51) (stroke (width 0.12) (type solid)) (layer "F.SilkS"))
  (pad "1" smd roundrect (at -0.775 0 90) (size 0.9 0.95) (layers "F.Cu" "F.Mask" "F.Paste") (roundrect_rratio 0.25) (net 1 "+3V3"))
  (pad "2" smd roundrect (at 0.775 0 90) (size 0.9 0.95) (layers "F.Cu" "F.Mask" "F.Paste") (roundrect_rratio 0.25) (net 3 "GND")))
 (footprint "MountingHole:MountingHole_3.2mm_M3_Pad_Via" (layer "F.Cu") (at 123.5 96.000002)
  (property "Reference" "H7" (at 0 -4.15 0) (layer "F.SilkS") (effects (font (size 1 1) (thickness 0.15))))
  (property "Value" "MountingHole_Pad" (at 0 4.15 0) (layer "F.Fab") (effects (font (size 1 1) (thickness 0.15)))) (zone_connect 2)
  (pad "1" thru_hole circle (at -2.4 0) (size 0.8 0.8) (drill 0.5) (layers "*.Cu" "*.Mask") (remove_unused_layers no) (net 3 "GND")
   (zone_connect 2))
  (pad "1" thru_hole circle (at -1.697056 -1.697056) (size 0.8 0.8) (drill 0.5) (layers "*.Cu" "*.Mask") (remove_unused_layers no)
   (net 3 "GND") (zone_connect 2))
  (pad "1" thru_hole circle (at -1.697056 1.697056) (size 0.8 0.8) (drill 0.5) (layers "*.Cu" "*.Mask") (remove_unused_layers no)
   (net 3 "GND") (zone_connect 2))
  (pad "1" thru_hole circle (at 0 -2.4) (size 0.8 0.8) (drill 0.5) (layers "*.Cu" "*.Mask") (remove_unused_layers no) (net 3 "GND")
   (zone_connect 2))
  (pad "1" thru_hole circle (at 0 0) (size 6.4 6.4) (drill 3.2) (layers "*.Cu" "*.Mask") (remove_unused_layers no) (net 3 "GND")
   (zone_connect 2))
  (pad "1" thru_hole circle (at 0 2.4) (size 0.8 0.8) (drill 0.5) (layers "*.Cu" "*.Mask") (remove_unused_layers no) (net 3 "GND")
   (zone_connect 2))
  (pad "1" thru_hole circle (at 1.697056 -1.697056) (size 0.8 0.8) (drill 0.5) (layers "*.Cu" "*.Mask") (remove_unused_layers no)
   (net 3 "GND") (zone_connect 2))
  (pad "1" thru_hole circle (at 1.697056 1.697056) (size 0.8 0.8) (drill 0.5) (layers "*.Cu" "*.Mask") (remove_unused_layers no)
   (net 3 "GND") (zone_connect 2))
  (pad "1" thru_hole circle (at 2.4 0) (size 0.8 0.8) (drill 0.5) (layers "*.Cu" "*.Mask") (remove_unused_layers no) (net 3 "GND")
   (zone_connect 2)))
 (gr_rect (start 120 68.5) (end 148 99.5) (stroke (width 0.05) (type default)) (fill no) (layer "Edge.Cuts"))
 (segment (start 141.3 85.6) (end 143.675 85.6) (width 0.2) (layer "F.Cu") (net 5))
 (segment (start 134.01 85.05) (end 140.75 85.05) (width 0.2) (layer "F.Cu") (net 5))
 (segment (start 140.75 85.05) (end 141.3 85.6) (width 0.2) (layer "F.Cu") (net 5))
 (segment (start 143.675 85.6) (end 143.815 85.46) (width 0.2) (layer "F.Cu") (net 5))
 (segment (start 134.01 83.79) (end 140.37 83.79) (width 0.2) (layer "F.Cu") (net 6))
 (segment (start 141.24 82.92) (end 143.815 82.92) (width 0.2) (layer "F.Cu") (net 6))
 (segment (start 140.37 83.79) (end 141.24 82.92) (width 0.2) (layer "F.Cu") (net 6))
 (segment (start 131.6 80.11) (end 134.01 82.52) (width 0.2) (layer "F.Cu") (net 7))
 (segment (start 131.6 79.2625) (end 131.6 80.11) (width 0.2) (layer "F.Cu") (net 7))
 (segment (start 128.59 86.32) (end 130.27 88) (width 0.2) (layer "F.Cu") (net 3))
 (segment (start 128.9 86.32) (end 128.59 86.32) (width 0.2) (layer "F.Cu") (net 3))
 (segment (start 130.3 79.2625) (end 130.3 84.92) (width 0.2) (layer "F.Cu") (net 3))
 (segment (start 130.3 84.92) (end 128.9 86.32) (width 0.2) (layer "F.Cu") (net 3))
 (segment (start 130.27 88) (end 143.815 88) (width 0.2) (layer "F.Cu") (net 3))
 (segment (start 129.9 77.12) (end 131.5125 77.12) (width 0.2) (layer "F.Cu") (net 1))
 (segment (start 131.5125 77.12) (end 132.9 78.5075) (width 0.2) (layer "F.Cu") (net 1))
 (segment (start 140.875 80.095) (end 141.88 81.1) (width 0.2) (layer "F.Cu") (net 1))
 (segment (start 142.5 81.1) (end 143.22 80.38) (width 0.2) (layer "F.Cu") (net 1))
 (segment (start 128.59 82.52) (end 128.59 78.43) (width 0.2) (layer "F.Cu") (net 1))
 (segment (start 132.9 79.2625) (end 132.9425 79.2625) (width 0.2) (layer "F.Cu") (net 1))
 (segment (start 133.775 80.095) (end 136.1 80.095) (width 0.2) (layer "F.Cu") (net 1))
 (segment (start 132.9425 79.2625) (end 133.775 80.095) (width 0.2) (layer "F.Cu") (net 1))
 (segment (start 128.59 78.43) (end 129.9 77.12) (width 0.2) (layer "F.Cu") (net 1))
 (segment (start 141.88 81.1) (end 142.5 81.1) (width 0.2) (layer "F.Cu") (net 1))
 (segment (start 138 80.095) (end 140.875 80.095) (width 0.2) (layer "F.Cu") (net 1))
 (segment (start 143.22 80.38) (end 143.815 80.38) (width 0.2) (layer "F.Cu") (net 1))
 (segment (start 128.59 83.79) (end 128.59 82.52) (width 0.2) (layer "F.Cu") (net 1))
 (segment (start 136.1 80.095) (end 138 80.095) (width 0.2) (layer "F.Cu") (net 1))
 (segment (start 132.9 78.5075) (end 132.9 79.2625) (width 0.2) (layer "F.Cu") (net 1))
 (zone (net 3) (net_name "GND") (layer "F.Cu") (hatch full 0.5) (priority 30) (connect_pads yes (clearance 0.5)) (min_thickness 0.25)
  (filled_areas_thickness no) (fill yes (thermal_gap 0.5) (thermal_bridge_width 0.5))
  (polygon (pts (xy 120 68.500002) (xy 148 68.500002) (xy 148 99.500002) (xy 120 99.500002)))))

